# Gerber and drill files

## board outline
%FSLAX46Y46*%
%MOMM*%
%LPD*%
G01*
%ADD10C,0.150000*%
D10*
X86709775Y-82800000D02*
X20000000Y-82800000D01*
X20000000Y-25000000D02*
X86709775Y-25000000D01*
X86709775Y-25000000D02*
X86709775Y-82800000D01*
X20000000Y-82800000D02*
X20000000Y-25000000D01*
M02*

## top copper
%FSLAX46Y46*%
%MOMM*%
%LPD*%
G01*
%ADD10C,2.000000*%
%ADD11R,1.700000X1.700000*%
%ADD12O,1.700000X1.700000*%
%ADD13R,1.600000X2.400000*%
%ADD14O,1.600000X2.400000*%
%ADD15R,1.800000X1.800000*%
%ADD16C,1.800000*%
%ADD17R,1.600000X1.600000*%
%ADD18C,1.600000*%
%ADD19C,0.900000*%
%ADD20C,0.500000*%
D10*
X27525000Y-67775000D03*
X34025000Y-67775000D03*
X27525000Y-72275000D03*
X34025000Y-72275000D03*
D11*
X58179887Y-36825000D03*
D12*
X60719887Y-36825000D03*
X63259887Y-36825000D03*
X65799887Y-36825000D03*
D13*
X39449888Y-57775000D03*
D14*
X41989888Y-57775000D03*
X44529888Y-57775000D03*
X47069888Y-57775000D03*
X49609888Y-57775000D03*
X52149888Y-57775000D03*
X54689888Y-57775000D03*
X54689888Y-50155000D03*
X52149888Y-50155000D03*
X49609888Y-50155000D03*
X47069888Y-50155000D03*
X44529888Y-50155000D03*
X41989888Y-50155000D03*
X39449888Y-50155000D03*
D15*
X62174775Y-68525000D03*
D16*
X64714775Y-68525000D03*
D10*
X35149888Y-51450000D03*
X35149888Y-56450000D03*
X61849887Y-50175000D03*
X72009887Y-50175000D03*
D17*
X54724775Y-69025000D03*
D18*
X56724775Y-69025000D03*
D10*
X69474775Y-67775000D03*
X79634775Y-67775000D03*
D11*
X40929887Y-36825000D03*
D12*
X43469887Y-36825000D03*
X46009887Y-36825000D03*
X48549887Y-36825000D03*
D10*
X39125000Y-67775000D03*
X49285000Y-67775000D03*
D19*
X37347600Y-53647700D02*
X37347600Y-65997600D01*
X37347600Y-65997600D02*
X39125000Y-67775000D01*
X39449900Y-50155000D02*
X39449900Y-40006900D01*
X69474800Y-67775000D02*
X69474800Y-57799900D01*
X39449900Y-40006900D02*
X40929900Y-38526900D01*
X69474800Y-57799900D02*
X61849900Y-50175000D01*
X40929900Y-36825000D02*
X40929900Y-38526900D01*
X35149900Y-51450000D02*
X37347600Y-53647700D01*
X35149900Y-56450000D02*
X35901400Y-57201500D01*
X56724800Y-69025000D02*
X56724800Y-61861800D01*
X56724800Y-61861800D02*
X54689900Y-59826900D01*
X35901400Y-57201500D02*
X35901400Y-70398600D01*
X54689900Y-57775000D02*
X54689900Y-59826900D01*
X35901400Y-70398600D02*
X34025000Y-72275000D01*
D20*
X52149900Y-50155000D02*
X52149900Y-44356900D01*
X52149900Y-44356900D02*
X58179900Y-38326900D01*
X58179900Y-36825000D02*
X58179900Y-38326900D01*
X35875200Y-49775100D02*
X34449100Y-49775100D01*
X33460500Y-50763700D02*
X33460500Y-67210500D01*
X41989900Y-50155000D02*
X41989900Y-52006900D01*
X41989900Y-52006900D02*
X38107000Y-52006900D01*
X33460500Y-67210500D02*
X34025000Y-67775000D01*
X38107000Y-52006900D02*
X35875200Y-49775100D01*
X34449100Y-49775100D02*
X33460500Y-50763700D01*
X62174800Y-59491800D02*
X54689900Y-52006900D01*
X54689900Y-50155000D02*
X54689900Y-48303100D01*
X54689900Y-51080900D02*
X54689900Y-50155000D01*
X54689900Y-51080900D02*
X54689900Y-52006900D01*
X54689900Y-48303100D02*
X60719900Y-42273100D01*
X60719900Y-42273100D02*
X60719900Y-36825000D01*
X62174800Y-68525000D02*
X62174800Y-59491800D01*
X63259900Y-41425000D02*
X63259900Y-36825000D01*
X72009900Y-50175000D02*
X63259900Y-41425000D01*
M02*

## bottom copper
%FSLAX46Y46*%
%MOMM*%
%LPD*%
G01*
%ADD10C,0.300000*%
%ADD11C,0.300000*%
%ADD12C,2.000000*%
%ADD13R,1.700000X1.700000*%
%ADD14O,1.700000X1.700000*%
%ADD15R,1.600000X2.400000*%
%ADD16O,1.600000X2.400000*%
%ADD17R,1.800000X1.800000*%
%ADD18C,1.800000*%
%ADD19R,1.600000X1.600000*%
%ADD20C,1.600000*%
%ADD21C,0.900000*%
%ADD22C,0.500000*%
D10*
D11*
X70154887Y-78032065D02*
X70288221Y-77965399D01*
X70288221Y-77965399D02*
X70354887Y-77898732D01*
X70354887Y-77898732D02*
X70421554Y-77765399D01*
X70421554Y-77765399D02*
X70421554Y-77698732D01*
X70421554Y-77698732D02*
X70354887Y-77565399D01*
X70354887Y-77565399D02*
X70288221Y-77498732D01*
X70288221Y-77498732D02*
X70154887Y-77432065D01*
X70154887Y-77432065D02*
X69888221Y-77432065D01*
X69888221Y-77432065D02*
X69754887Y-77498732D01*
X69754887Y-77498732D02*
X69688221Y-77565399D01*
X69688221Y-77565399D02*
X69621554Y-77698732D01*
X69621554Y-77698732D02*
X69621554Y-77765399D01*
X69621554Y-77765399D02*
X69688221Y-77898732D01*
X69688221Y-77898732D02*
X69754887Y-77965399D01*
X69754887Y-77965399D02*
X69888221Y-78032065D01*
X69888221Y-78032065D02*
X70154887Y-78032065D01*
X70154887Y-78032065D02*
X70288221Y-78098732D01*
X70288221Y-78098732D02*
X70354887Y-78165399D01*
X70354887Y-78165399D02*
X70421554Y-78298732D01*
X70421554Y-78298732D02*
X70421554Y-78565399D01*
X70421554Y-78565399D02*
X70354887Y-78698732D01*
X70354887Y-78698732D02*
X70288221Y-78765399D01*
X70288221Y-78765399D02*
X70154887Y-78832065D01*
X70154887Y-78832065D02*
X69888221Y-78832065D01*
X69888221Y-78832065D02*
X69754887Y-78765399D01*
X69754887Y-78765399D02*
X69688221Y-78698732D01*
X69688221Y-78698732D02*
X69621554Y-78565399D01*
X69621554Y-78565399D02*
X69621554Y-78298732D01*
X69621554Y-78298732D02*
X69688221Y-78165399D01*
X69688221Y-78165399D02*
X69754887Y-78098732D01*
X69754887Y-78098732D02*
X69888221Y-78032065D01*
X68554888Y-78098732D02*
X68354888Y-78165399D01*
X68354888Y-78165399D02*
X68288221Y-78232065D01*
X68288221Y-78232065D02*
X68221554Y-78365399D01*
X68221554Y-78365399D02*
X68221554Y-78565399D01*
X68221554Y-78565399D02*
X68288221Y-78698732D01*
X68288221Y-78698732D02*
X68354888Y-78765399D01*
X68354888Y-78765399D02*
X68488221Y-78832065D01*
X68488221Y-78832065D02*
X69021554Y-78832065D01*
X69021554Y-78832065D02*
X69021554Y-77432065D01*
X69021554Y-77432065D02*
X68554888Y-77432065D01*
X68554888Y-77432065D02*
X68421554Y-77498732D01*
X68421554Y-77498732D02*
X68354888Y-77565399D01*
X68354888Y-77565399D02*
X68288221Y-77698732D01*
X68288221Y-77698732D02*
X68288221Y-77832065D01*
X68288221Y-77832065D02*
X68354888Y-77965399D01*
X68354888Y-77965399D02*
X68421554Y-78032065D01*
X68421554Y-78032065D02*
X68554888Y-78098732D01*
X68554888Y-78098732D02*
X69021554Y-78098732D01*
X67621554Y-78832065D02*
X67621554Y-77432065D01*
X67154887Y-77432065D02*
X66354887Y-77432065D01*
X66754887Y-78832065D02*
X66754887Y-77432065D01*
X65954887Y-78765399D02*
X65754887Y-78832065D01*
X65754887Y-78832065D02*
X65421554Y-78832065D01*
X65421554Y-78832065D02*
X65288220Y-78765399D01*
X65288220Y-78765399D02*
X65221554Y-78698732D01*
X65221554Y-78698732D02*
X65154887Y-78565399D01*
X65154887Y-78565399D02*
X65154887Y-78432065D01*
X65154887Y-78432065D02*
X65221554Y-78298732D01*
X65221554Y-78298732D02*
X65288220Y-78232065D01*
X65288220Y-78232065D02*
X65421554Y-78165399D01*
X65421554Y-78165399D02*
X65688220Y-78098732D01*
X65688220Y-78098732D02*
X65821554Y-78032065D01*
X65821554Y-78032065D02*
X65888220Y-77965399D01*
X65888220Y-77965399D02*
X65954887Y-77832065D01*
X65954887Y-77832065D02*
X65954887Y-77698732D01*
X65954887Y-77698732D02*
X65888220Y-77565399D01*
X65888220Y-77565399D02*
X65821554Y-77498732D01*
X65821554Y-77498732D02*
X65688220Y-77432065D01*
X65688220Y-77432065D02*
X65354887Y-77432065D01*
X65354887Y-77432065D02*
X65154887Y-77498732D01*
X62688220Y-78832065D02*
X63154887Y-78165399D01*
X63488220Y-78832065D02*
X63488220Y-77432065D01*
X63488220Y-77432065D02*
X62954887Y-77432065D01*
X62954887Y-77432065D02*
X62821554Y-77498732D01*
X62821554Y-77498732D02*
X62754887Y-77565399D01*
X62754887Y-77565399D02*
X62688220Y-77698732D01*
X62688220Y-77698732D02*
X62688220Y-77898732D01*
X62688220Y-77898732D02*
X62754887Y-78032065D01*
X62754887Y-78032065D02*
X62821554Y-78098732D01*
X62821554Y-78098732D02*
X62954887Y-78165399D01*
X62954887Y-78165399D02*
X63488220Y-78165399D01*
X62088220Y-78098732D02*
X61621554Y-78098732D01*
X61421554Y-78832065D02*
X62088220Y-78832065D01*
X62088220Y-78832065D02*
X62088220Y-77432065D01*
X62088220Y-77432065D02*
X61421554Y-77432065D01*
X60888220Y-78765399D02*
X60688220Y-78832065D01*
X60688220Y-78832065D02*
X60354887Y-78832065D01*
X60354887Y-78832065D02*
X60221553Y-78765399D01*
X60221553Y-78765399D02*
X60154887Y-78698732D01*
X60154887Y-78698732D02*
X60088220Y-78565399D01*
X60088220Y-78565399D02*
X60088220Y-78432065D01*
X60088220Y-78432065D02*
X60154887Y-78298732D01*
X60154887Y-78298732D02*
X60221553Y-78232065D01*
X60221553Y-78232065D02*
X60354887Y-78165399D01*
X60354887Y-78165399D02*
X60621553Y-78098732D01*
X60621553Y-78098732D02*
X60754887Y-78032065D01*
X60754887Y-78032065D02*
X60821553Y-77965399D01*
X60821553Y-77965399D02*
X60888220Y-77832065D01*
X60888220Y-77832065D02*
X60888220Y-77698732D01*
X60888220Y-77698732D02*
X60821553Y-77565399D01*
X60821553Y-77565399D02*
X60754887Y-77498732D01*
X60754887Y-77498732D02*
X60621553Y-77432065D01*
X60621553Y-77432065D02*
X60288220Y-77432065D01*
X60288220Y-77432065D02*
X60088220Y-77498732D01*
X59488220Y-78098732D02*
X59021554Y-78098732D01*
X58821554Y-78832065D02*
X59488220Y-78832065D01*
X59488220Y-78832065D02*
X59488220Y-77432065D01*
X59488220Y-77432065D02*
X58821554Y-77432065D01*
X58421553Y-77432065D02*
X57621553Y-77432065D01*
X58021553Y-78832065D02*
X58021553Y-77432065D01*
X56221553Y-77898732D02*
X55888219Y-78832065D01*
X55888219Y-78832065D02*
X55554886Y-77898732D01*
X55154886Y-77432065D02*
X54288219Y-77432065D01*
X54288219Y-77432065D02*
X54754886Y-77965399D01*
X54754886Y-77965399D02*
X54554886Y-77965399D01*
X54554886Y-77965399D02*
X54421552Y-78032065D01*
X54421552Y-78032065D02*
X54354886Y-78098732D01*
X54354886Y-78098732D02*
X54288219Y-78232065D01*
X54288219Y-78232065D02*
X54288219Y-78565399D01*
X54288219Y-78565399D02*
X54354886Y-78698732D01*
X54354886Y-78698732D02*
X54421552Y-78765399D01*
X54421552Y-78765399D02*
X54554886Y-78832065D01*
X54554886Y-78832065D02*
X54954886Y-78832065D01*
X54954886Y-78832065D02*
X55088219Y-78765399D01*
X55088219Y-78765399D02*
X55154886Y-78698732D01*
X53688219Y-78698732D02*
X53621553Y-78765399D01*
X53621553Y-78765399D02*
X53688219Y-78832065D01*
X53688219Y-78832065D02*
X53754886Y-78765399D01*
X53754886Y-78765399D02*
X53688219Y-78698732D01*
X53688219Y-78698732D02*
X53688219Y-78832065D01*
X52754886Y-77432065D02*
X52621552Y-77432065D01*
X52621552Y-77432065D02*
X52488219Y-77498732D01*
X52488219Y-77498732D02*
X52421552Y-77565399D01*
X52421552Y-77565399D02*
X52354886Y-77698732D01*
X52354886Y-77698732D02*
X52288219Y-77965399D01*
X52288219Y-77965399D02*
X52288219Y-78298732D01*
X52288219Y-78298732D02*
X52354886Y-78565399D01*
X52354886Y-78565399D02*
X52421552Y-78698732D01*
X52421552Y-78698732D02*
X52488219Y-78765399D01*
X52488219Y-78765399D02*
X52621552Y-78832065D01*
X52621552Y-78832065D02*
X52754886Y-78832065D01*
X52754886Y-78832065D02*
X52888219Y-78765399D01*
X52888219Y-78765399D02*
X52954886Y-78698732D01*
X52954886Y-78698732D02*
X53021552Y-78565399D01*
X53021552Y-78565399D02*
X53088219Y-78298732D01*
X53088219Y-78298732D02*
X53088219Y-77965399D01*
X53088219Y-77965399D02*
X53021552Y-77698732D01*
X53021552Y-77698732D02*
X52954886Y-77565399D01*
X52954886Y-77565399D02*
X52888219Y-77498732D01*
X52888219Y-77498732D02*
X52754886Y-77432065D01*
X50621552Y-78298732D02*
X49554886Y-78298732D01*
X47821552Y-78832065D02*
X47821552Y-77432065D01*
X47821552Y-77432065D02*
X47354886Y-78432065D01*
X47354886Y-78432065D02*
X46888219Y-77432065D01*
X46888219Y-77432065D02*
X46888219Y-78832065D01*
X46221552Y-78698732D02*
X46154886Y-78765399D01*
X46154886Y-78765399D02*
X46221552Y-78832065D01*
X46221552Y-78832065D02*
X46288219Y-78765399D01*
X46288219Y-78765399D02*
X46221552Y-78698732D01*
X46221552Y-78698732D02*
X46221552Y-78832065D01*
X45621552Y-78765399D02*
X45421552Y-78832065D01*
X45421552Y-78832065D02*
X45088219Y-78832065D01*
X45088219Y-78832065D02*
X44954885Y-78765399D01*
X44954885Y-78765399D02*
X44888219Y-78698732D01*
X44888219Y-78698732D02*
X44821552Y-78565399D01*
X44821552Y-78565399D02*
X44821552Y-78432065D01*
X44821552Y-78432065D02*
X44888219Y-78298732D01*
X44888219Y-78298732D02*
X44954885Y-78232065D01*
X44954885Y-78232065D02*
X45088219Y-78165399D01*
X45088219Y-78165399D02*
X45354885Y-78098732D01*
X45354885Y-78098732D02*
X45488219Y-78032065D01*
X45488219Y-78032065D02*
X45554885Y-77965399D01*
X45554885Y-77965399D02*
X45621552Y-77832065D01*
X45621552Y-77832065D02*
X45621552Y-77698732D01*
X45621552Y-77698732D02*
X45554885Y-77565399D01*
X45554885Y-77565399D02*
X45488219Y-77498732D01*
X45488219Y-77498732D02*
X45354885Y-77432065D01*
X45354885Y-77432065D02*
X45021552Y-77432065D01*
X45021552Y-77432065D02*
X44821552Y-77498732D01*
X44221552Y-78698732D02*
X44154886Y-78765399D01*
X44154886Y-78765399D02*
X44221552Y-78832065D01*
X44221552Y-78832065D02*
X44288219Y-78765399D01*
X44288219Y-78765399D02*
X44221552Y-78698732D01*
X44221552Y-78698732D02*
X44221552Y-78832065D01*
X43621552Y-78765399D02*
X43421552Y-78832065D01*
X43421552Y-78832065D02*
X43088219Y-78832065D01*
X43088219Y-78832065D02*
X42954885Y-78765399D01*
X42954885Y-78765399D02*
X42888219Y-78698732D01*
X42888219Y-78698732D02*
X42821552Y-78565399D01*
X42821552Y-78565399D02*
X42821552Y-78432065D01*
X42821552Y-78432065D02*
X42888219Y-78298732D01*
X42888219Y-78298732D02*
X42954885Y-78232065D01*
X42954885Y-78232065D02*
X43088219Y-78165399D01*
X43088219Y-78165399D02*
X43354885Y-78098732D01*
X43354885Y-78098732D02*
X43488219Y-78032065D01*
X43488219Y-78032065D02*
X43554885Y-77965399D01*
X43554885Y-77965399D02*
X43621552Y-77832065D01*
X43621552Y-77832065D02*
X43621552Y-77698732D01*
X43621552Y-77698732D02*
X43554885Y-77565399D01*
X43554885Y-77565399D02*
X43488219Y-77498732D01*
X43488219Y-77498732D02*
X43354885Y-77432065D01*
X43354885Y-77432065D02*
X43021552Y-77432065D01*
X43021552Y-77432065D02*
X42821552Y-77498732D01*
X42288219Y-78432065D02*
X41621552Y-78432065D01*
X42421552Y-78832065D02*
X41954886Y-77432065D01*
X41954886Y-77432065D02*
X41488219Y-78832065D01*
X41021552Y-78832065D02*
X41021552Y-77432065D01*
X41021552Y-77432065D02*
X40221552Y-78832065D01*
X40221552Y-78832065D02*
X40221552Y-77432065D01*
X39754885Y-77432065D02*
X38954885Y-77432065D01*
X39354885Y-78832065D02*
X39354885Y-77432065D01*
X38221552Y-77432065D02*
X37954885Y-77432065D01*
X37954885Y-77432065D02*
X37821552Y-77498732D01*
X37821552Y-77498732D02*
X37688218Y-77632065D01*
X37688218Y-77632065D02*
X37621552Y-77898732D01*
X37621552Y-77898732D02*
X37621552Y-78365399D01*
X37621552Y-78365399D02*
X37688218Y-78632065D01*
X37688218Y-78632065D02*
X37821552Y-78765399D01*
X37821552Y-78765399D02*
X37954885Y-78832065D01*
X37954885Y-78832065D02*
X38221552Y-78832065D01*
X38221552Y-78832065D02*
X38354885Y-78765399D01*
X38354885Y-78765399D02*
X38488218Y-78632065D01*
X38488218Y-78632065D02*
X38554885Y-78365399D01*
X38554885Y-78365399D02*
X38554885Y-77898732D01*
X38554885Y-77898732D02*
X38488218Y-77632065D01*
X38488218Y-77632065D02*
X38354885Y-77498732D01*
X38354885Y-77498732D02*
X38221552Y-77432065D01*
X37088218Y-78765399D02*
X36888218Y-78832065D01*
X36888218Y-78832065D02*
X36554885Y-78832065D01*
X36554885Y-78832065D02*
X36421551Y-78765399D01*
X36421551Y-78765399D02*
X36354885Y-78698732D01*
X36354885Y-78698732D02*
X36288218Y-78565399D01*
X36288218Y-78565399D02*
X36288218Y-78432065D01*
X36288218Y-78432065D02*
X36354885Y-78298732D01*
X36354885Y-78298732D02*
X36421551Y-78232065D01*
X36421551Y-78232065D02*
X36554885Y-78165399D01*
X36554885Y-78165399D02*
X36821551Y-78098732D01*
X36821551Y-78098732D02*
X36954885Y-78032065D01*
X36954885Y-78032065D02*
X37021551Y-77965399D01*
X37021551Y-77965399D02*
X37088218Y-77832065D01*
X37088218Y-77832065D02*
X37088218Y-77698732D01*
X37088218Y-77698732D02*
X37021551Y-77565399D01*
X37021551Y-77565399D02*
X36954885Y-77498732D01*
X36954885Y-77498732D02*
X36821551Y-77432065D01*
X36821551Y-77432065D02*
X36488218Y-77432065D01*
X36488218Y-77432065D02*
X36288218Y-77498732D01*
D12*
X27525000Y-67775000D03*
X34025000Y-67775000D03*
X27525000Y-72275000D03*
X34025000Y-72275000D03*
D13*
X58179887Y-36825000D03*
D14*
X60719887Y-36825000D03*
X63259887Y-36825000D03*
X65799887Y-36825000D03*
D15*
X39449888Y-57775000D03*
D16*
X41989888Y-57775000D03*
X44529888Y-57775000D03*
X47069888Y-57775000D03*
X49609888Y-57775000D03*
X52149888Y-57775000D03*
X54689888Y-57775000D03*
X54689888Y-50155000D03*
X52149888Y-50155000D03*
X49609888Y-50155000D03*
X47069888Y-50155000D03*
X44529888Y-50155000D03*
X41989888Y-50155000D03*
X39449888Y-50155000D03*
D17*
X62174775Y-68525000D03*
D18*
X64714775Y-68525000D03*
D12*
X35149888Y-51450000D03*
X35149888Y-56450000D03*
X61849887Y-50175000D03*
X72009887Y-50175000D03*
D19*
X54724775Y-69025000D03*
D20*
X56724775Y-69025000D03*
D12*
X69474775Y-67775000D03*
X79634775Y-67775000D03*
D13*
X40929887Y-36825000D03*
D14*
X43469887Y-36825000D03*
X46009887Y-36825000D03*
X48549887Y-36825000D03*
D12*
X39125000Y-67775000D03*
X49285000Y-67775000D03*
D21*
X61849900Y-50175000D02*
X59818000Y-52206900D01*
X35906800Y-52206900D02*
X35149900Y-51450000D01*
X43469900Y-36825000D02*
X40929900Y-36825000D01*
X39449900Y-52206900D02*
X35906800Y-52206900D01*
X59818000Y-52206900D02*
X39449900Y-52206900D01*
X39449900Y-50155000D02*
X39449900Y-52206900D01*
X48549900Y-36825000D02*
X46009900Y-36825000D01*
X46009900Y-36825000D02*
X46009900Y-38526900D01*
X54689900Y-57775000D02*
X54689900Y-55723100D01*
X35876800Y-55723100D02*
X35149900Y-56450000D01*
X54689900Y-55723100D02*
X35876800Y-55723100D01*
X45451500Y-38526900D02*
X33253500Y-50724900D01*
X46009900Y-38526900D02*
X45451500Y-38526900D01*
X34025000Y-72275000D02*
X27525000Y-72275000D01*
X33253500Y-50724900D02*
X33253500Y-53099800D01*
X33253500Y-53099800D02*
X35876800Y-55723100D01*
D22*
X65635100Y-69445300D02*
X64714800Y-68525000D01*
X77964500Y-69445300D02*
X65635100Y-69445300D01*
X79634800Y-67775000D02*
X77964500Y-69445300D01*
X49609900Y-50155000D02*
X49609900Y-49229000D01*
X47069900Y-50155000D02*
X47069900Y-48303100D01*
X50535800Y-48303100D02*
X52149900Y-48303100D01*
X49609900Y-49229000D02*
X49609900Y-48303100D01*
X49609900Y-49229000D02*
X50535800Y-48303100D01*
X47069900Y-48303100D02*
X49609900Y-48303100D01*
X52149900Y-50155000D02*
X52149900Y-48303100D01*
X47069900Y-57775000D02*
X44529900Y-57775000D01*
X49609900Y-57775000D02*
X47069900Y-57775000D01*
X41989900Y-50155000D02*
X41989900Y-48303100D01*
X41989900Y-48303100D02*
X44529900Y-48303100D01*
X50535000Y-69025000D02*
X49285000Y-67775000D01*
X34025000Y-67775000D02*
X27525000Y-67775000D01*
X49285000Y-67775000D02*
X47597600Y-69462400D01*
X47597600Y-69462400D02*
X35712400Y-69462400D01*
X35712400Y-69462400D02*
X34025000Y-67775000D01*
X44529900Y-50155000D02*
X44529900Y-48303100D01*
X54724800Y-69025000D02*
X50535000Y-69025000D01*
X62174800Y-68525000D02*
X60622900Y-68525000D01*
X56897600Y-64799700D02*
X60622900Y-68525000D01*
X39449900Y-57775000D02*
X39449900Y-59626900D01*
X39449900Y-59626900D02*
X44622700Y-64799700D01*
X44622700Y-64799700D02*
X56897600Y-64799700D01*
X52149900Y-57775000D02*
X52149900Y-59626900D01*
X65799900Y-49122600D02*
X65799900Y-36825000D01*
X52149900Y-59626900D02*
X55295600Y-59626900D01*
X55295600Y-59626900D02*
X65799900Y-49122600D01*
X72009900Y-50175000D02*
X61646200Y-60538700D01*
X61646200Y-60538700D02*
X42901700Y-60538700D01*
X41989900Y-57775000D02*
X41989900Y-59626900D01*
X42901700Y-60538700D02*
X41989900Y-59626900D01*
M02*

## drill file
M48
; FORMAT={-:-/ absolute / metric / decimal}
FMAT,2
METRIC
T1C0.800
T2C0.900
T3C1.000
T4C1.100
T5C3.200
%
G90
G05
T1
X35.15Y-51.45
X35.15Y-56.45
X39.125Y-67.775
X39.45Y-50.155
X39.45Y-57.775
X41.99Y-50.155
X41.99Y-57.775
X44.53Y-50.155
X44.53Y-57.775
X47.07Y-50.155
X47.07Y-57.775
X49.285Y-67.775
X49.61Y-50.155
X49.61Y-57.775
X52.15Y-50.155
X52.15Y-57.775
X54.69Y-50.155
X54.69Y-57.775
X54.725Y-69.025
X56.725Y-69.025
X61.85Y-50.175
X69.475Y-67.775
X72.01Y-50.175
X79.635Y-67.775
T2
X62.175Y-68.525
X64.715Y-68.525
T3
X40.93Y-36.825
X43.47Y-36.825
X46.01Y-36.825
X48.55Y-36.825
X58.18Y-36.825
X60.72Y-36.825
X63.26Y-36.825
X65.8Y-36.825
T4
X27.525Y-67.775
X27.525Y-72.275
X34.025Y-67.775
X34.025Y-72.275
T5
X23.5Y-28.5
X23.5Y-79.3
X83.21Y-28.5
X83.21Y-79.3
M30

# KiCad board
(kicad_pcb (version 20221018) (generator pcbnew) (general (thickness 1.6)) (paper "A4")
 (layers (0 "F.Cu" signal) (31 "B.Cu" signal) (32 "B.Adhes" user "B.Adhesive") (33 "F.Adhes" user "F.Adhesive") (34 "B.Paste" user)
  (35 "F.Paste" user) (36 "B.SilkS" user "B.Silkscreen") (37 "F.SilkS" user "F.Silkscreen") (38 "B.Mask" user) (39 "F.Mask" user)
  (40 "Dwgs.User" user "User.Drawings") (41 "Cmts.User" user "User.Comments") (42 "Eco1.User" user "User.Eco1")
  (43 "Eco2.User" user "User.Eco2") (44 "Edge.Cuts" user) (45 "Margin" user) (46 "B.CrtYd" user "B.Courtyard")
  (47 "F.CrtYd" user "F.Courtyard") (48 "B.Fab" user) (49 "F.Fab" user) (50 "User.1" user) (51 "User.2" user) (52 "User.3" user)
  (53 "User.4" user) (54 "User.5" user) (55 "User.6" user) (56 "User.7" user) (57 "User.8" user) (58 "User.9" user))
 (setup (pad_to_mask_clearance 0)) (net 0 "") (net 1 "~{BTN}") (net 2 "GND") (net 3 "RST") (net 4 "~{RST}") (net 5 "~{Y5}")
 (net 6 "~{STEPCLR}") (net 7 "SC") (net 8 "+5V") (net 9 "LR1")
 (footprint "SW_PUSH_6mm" (layer "F.Cu") (at 27.525 67.775)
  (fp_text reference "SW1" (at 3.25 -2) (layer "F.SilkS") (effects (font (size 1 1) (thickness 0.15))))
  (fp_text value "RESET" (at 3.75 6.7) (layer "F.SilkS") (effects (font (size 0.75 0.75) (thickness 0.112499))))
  (pad "1" thru_hole circle (at 0 0 90) (size 2 2) (drill 1.1) (layers "F&B.Cu" "*.Mask") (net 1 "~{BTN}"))
  (pad "1" thru_hole circle (at 6.5 0 90) (size 2 2) (drill 1.1) (layers "F&B.Cu" "*.Mask") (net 1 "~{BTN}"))
  (pad "2" thru_hole circle (at 0 4.5 90) (size 2 2) (drill 1.1) (layers "F&B.Cu" "*.Mask") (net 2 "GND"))
  (pad "2" thru_hole circle (at 6.5 4.5 90) (size 2 2) (drill 1.1) (layers "F&B.Cu" "*.Mask") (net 2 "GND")))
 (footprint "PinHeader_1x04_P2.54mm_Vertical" (layer "F.Cu") (at 58.179887 36.825 90)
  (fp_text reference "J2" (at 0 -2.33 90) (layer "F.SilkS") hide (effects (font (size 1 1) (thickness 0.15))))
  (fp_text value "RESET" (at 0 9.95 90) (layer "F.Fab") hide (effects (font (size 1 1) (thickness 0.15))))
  (pad "1" thru_hole rect (at 0 0 90) (size 1.7 1.7) (drill 1) (layers "F&B.Cu" "*.Mask") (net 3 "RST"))
  (pad "2" thru_hole oval (at 0 2.54 90) (size 1.7 1.7) (drill 1) (layers "F&B.Cu" "*.Mask") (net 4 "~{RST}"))
  (pad "3" thru_hole oval (at 0 5.08 90) (size 1.7 1.7) (drill 1) (layers "F&B.Cu" "*.Mask") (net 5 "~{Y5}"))
  (pad "4" thru_hole oval (at 0 7.62 90) (size 1.7 1.7) (drill 1) (layers "F&B.Cu" "*.Mask") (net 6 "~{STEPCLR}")))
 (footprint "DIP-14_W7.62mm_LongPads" (layer "F.Cu") (at 39.449888 57.775 90)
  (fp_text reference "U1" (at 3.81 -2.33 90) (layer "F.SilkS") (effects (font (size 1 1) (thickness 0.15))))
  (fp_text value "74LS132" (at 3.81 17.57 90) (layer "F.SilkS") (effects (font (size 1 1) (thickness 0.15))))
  (pad "1" thru_hole rect (at 0 0 90) (size 2.4 1.6) (drill 0.8) (layers "F&B.Cu" "*.Mask") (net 4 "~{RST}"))
  (pad "2" thru_hole oval (at 0 2.54 90) (size 2.4 1.6) (drill 0.8) (layers "F&B.Cu" "*.Mask") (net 5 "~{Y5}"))
  (pad "3" thru_hole oval (at 0 5.08 90) (size 2.4 1.6) (drill 0.8) (layers "F&B.Cu" "*.Mask") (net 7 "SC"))
  (pad "4" thru_hole oval (at 0 7.62 90) (size 2.4 1.6) (drill 0.8) (layers "F&B.Cu" "*.Mask") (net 7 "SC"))
  (pad "5" thru_hole oval (at 0 10.16 90) (size 2.4 1.6) (drill 0.8) (layers "F&B.Cu" "*.Mask") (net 7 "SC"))
  (pad "6" thru_hole oval (at 0 12.7 90) (size 2.4 1.6) (drill 0.8) (layers "F&B.Cu" "*.Mask") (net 6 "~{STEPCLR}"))
  (pad "7" thru_hole oval (at 0 15.24 90) (size 2.4 1.6) (drill 0.8) (layers "F&B.Cu" "*.Mask") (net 2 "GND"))
  (pad "8" thru_hole oval (at 7.62 15.24 90) (size 2.4 1.6) (drill 0.8) (layers "F&B.Cu" "*.Mask") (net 4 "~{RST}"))
  (pad "9" thru_hole oval (at 7.62 12.7 90) (size 2.4 1.6) (drill 0.8) (layers "F&B.Cu" "*.Mask") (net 3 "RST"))
  (pad "10" thru_hole oval (at 7.62 10.16 90) (size 2.4 1.6) (drill 0.8) (layers "F&B.Cu" "*.Mask") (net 3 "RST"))
  (pad "11" thru_hole oval (at 7.62 7.62 90) (size 2.4 1.6) (drill 0.8) (layers "F&B.Cu" "*.Mask") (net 3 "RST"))
  (pad "12" thru_hole oval (at 7.62 5.08 90) (size 2.4 1.6) (drill 0.8) (layers "F&B.Cu" "*.Mask") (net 1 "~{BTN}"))
  (pad "13" thru_hole oval (at 7.62 2.54 90) (size 2.4 1.6) (drill 0.8) (layers "F&B.Cu" "*.Mask") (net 1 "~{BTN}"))
  (pad "14" thru_hole oval (at 7.62 0 90) (size 2.4 1.6) (drill 0.8) (layers "F&B.Cu" "*.Mask") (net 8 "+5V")))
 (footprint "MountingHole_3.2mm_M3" (layer "F.Cu") (at 23.5 79.3)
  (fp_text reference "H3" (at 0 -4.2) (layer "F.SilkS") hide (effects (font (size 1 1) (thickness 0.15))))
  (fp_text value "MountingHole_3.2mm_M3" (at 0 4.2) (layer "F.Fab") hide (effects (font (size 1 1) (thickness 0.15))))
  (pad "" np_thru_hole circle (at 0 0) (size 3.2 3.2) (drill 3.2) (layers "*.Cu" "*.Mask")))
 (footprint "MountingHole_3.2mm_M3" (layer "F.Cu") (at 83.209775 79.3)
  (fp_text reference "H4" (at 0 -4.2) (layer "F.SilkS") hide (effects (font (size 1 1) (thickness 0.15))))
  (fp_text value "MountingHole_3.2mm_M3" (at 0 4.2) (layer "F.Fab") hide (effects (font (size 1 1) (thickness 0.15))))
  (pad "" np_thru_hole circle (at 0 0) (size 3.2 3.2) (drill 3.2) (layers "*.Cu" "*.Mask")))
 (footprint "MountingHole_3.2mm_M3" (layer "F.Cu") (at 83.209775 28.5)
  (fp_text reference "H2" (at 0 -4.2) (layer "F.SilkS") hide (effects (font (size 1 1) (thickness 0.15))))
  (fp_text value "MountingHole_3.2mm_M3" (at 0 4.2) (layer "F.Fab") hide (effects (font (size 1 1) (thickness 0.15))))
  (pad "" np_thru_hole circle (at 0 0) (size 3.2 3.2) (drill 3.2) (layers "*.Cu" "*.Mask")))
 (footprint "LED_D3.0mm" (layer "F.Cu") (at 62.174775 68.525)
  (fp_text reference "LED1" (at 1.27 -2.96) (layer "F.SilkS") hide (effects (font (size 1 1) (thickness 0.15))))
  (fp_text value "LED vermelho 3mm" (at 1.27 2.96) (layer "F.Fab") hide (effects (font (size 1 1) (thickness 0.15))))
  (pad "1" thru_hole rect (at 0 0) (size 1.8 1.8) (drill 0.9) (layers "F&B.Cu" "*.Mask") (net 4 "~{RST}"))
  (pad "2" thru_hole circle (at 2.54 0) (size 1.8 1.8) (drill 0.9) (layers "F&B.Cu" "*.Mask") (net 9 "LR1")))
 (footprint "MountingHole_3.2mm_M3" (layer "F.Cu") (at 23.5 28.5)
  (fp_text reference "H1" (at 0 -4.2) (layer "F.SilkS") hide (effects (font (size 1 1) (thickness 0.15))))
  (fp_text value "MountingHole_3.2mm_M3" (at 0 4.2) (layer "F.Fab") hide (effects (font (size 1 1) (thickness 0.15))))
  (pad "" np_thru_hole circle (at 0 0) (size 3.2 3.2) (drill 3.2) (layers "*.Cu" "*.Mask")))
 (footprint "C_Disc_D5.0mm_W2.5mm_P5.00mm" (layer "F.Cu") (at 35.149888 51.45 -90)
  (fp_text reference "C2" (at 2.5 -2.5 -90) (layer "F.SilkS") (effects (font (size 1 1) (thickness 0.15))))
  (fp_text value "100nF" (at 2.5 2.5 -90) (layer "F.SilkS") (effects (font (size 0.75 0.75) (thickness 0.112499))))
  (pad "1" thru_hole circle (at 0 0 270) (size 2 2) (drill 0.8) (layers "F&B.Cu" "*.Mask") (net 8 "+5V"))
  (pad "2" thru_hole circle (at 5 0 270) (size 2 2) (drill 0.8) (layers "F&B.Cu" "*.Mask") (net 2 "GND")))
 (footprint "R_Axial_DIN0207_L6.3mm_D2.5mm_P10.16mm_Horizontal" (layer "F.Cu") (at 61.849887 50.175)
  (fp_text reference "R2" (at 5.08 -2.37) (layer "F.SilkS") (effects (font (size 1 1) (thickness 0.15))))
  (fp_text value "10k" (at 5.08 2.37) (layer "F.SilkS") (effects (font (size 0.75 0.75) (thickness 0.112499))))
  (pad "1" thru_hole circle (at 0 0) (size 2 2) (drill 0.8) (layers "F&B.Cu" "*.Mask") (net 8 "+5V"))
  (pad "2" thru_hole circle (at 10.16 0) (size 2 2) (drill 0.8) (layers "F&B.Cu" "*.Mask") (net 5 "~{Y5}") (thermal_bridge_angle 90)))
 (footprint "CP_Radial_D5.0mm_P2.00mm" (layer "F.Cu") (at 54.724775 69.025)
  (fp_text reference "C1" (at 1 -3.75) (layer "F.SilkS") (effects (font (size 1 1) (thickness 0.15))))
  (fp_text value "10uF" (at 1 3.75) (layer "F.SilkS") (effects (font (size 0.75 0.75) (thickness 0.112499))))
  (pad "1" thru_hole rect (at 0 0) (size 1.6 1.6) (drill 0.8) (layers "F&B.Cu" "*.Mask") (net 1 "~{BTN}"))
  (pad "2" thru_hole circle (at 2 0) (size 1.6 1.6) (drill 0.8) (layers "F&B.Cu" "*.Mask") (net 2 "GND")))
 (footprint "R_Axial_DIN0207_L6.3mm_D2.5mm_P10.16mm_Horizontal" (layer "F.Cu") (at 69.474775 67.775)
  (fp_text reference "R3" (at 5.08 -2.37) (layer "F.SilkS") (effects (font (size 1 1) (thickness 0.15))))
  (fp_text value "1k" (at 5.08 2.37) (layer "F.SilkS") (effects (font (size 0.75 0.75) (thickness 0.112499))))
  (pad "1" thru_hole circle (at 0 0) (size 2 2) (drill 0.8) (layers "F&B.Cu" "*.Mask") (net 8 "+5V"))
  (pad "2" thru_hole circle (at 10.16 0) (size 2 2) (drill 0.8) (layers "F&B.Cu" "*.Mask") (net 9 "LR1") (thermal_bridge_angle 90)))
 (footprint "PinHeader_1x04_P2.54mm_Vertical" (layer "F.Cu") (at 40.929887 36.825 90)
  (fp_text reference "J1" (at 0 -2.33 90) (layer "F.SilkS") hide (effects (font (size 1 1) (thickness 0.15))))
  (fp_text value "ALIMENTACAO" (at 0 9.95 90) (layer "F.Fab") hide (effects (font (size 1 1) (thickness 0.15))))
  (pad "1" thru_hole rect (at 0 0 90) (size 1.7 1.7) (drill 1) (layers "F&B.Cu" "*.Mask") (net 8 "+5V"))
  (pad "2" thru_hole oval (at 0 2.54 90) (size 1.7 1.7) (drill 1) (layers "F&B.Cu" "*.Mask") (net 8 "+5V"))
  (pad "3" thru_hole oval (at 0 5.08 90) (size 1.7 1.7) (drill 1) (layers "F&B.Cu" "*.Mask") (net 2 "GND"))
  (pad "4" thru_hole oval (at 0 7.62 90) (size 1.7 1.7) (drill 1) (layers "F&B.Cu" "*.Mask") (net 2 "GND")))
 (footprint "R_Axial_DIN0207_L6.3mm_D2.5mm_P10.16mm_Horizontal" (layer "F.Cu") (at 39.125 67.775)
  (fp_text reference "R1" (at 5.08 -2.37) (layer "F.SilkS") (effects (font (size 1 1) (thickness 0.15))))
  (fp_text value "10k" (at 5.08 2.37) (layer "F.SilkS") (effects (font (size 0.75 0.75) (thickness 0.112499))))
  (pad "1" thru_hole circle (at 0 0) (size 2 2) (drill 0.8) (layers "F&B.Cu" "*.Mask") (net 8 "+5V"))
  (pad "2" thru_hole circle (at 10.16 0) (size 2 2) (drill 0.8) (layers "F&B.Cu" "*.Mask") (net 1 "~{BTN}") (thermal_bridge_angle 90)))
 (gr_line (start 86.709775 82.8) (end 20 82.8) (stroke (width 0.15) (type default)) (layer "Edge.Cuts"))
 (gr_line (start 20 25) (end 86.709775 25) (stroke (width 0.15) (type default)) (layer "Edge.Cuts"))
 (gr_line (start 86.709775 25) (end 86.709775 82.8) (stroke (width 0.15) (type default)) (layer "Edge.Cuts"))
 (gr_line (start 20 82.8) (end 20 25) (stroke (width 0.15) (type default)) (layer "Edge.Cuts"))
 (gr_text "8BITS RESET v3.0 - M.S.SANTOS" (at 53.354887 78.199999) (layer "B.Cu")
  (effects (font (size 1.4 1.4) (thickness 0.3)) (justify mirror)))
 (segment (start 37.3476 53.6477) (end 37.3476 65.9976) (width 0.9) (layer "F.Cu") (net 8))
 (segment (start 37.3476 65.9976) (end 39.125 67.775) (width 0.9) (layer "F.Cu") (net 8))
 (segment (start 39.4499 50.155) (end 39.4499 40.0069) (width 0.9) (layer "F.Cu") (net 8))
 (segment (start 69.4748 67.775) (end 69.4748 57.7999) (width 0.9) (layer "F.Cu") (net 8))
 (segment (start 39.4499 40.0069) (end 40.9299 38.5269) (width 0.9) (layer "F.Cu") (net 8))
 (segment (start 69.4748 57.7999) (end 61.8499 50.175) (width 0.9) (layer "F.Cu") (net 8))
 (segment (start 40.9299 36.825) (end 40.9299 38.5269) (width 0.9) (layer "F.Cu") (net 8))
 (segment (start 35.1499 51.45) (end 37.3476 53.6477) (width 0.9) (layer "F.Cu") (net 8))
 (segment (start 61.8499 50.175) (end 59.818 52.2069) (width 0.9) (layer "B.Cu") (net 8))
 (segment (start 35.9068 52.2069) (end 35.1499 51.45) (width 0.9) (layer "B.Cu") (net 8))
 (segment (start 43.4699 36.825) (end 40.9299 36.825) (width 0.9) (layer "B.Cu") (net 8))
 (segment (start 39.4499 52.2069) (end 35.9068 52.2069) (width 0.9) (layer "B.Cu") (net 8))
 (segment (start 59.818 52.2069) (end 39.4499 52.2069) (width 0.9) (layer "B.Cu") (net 8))
 (segment (start 39.4499 50.155) (end 39.4499 52.2069) (width 0.9) (layer "B.Cu") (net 8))
 (segment (start 35.1499 56.45) (end 35.9014 57.2015) (width 0.9) (layer "F.Cu") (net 2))
 (segment (start 56.7248 69.025) (end 56.7248 61.8618) (width 0.9) (layer "F.Cu") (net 2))
 (segment (start 56.7248 61.8618) (end 54.6899 59.8269) (width 0.9) (layer "F.Cu") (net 2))
 (segment (start 35.9014 57.2015) (end 35.9014 70.3986) (width 0.9) (layer "F.Cu") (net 2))
 (segment (start 54.6899 57.775) (end 54.6899 59.8269) (width 0.9) (layer "F.Cu") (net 2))
 (segment (start 35.9014 70.3986) (end 34.025 72.275) (width 0.9) (layer "F.Cu") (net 2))
 (segment (start 48.5499 36.825) (end 46.0099 36.825) (width 0.9) (layer "B.Cu") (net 2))
 (segment (start 46.0099 36.825) (end 46.0099 38.5269) (width 0.9) (layer "B.Cu") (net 2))
 (segment (start 54.6899 57.775) (end 54.6899 55.7231) (width 0.9) (layer "B.Cu") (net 2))
 (segment (start 35.8768 55.7231) (end 35.1499 56.45) (width 0.9) (layer "B.Cu") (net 2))
 (segment (start 54.6899 55.7231) (end 35.8768 55.7231) (width 0.9) (layer "B.Cu") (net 2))
 (segment (start 45.4515 38.5269) (end 33.2535 50.7249) (width 0.9) (layer "B.Cu") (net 2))
 (segment (start 46.0099 38.5269) (end 45.4515 38.5269) (width 0.9) (layer "B.Cu") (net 2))
 (segment (start 34.025 72.275) (end 27.525 72.275) (width 0.9) (layer "B.Cu") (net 2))
 (segment (start 33.2535 50.7249) (end 33.2535 53.0998) (width 0.9) (layer "B.Cu") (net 2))
 (segment (start 33.2535 53.0998) (end 35.8768 55.7231) (width 0.9) (layer "B.Cu") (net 2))
 (segment (start 65.6351 69.4453) (end 64.7148 68.525) (width 0.5) (layer "B.Cu") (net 9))
 (segment (start 77.9645 69.4453) (end 65.6351 69.4453) (width 0.5) (layer "B.Cu") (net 9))
 (segment (start 79.6348 67.775) (end 77.9645 69.4453) (width 0.5) (layer "B.Cu") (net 9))
 (segment (start 52.1499 50.155) (end 52.1499 44.3569) (width 0.5) (layer "F.Cu") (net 3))
 (segment (start 52.1499 44.3569) (end 58.1799 38.3269) (width 0.5) (layer "F.Cu") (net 3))
 (segment (start 58.1799 36.825) (end 58.1799 38.3269) (width 0.5) (layer "F.Cu") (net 3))
 (segment (start 49.6099 50.155) (end 49.6099 49.229) (width 0.5) (layer "B.Cu") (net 3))
 (segment (start 47.0699 50.155) (end 47.0699 48.3031) (width 0.5) (layer "B.Cu") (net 3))
 (segment (start 50.5358 48.3031) (end 52.1499 48.3031) (width 0.5) (layer "B.Cu") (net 3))
 (segment (start 49.6099 49.229) (end 49.6099 48.3031) (width 0.5) (layer "B.Cu") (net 3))
 (segment (start 49.6099 49.229) (end 50.5358 48.3031) (width 0.5) (layer "B.Cu") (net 3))
 (segment (start 47.0699 48.3031) (end 49.6099 48.3031) (width 0.5) (layer "B.Cu") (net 3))
 (segment (start 52.1499 50.155) (end 52.1499 48.3031) (width 0.5) (layer "B.Cu") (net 3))
 (segment (start 47.0699 57.775) (end 44.5299 57.775) (width 0.5) (layer "B.Cu") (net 7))
 (segment (start 49.6099 57.775) (end 47.0699 57.775) (width 0.5) (layer "B.Cu") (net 7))
 (segment (start 35.8752 49.7751) (end 34.4491 49.7751) (width 0.5) (layer "F.Cu") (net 1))
 (segment (start 33.4605 50.7637) (end 33.4605 67.2105) (width 0.5) (layer "F.Cu") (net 1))
 (segment (start 41.9899 50.155) (end 41.9899 52.0069) (width 0.5) (layer "F.Cu") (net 1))
 (segment (start 41.9899 52.0069) (end 38.107 52.0069) (width 0.5) (layer "F.Cu") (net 1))
 (segment (start 33.4605 67.2105) (end 34.025 67.775) (width 0.5) (layer "F.Cu") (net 1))
 (segment (start 38.107 52.0069) (end 35.8752 49.7751) (width 0.5) (layer "F.Cu") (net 1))
 (segment (start 34.4491 49.7751) (end 33.4605 50.7637) (width 0.5) (layer "F.Cu") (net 1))
 (segment (start 41.9899 50.155) (end 41.9899 48.3031) (width 0.5) (layer "B.Cu") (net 1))
 (segment (start 41.9899 48.3031) (end 44.5299 48.3031) (width 0.5) (layer "B.Cu") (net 1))
 (segment (start 50.535 69.025) (end 49.285 67.775) (width 0.5) (layer "B.Cu") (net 1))
 (segment (start 34.025 67.775) (end 27.525 67.775) (width 0.5) (layer "B.Cu") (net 1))
 (segment (start 49.285 67.775) (end 47.5976 69.4624) (width 0.5) (layer "B.Cu") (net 1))
 (segment (start 47.5976 69.4624) (end 35.7124 69.4624) (width 0.5) (layer "B.Cu") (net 1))
 (segment (start 35.7124 69.4624) (end 34.025 67.775) (width 0.5) (layer "B.Cu") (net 1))
 (segment (start 44.5299 50.155) (end 44.5299 48.3031) (width 0.5) (layer "B.Cu") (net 1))
 (segment (start 54.7248 69.025) (end 50.535 69.025) (width 0.5) (layer "B.Cu") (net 1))
 (segment (start 62.1748 59.4918) (end 54.6899 52.0069) (width 0.5) (layer "F.Cu") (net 4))
 (segment (start 54.6899 50.155) (end 54.6899 48.3031) (width 0.5) (layer "F.Cu") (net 4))
 (segment (start 54.6899 51.0809) (end 54.6899 50.155) (width 0.5) (layer "F.Cu") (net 4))
 (segment (start 54.6899 51.0809) (end 54.6899 52.0069) (width 0.5) (layer "F.Cu") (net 4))
 (segment (start 54.6899 48.3031) (end 60.7199 42.2731) (width 0.5) (layer "F.Cu") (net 4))
 (segment (start 60.7199 42.2731) (end 60.7199 36.825) (width 0.5) (layer "F.Cu") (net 4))
 (segment (start 62.1748 68.525) (end 62.1748 59.4918) (width 0.5) (layer "F.Cu") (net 4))
 (segment (start 62.1748 68.525) (end 60.6229 68.525) (width 0.5) (layer "B.Cu") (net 4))
 (segment (start 56.8976 64.7997) (end 60.6229 68.525) (width 0.5) (layer "B.Cu") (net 4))
 (segment (start 39.4499 57.775) (end 39.4499 59.6269) (width 0.5) (layer "B.Cu") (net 4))
 (segment (start 39.4499 59.6269) (end 44.6227 64.7997) (width 0.5) (layer "B.Cu") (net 4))
 (segment (start 44.6227 64.7997) (end 56.8976 64.7997) (width 0.5) (layer "B.Cu") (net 4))
 (segment (start 52.1499 57.775) (end 52.1499 59.6269) (width 0.5) (layer "B.Cu") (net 6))
 (segment (start 65.7999 49.1226) (end 65.7999 36.825) (width 0.5) (layer "B.Cu") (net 6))
 (segment (start 52.1499 59.6269) (end 55.2956 59.6269) (width 0.5) (layer "B.Cu") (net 6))
 (segment (start 55.2956 59.6269) (end 65.7999 49.1226) (width 0.5) (layer "B.Cu") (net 6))
 (segment (start 63.2599 41.425) (end 63.2599 36.825) (width 0.5) (layer "F.Cu") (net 5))
 (segment (start 72.0099 50.175) (end 63.2599 41.425) (width 0.5) (layer "F.Cu") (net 5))
 (segment (start 72.0099 50.175) (end 61.6462 60.5387) (width 0.5) (layer "B.Cu") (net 5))
 (segment (start 61.6462 60.5387) (end 42.9017 60.5387) (width 0.5) (layer "B.Cu") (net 5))
 (segment (start 41.9899 57.775) (end 41.9899 59.6269) (width 0.5) (layer "B.Cu") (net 5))
 (segment (start 42.9017 60.5387) (end 41.9899 59.6269) (width 0.5) (layer "B.Cu") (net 5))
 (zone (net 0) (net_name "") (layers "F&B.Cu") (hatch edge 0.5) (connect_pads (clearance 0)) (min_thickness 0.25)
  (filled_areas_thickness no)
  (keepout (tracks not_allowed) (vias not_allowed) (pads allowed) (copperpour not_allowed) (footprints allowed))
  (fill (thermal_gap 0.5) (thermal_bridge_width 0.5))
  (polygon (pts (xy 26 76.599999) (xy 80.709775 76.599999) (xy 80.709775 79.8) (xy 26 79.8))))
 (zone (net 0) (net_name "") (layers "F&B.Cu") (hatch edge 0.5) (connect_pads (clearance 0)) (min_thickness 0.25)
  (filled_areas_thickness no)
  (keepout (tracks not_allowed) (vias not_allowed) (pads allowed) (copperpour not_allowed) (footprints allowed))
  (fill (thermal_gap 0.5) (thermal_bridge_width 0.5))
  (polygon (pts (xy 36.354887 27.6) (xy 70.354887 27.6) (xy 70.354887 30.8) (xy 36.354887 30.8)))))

